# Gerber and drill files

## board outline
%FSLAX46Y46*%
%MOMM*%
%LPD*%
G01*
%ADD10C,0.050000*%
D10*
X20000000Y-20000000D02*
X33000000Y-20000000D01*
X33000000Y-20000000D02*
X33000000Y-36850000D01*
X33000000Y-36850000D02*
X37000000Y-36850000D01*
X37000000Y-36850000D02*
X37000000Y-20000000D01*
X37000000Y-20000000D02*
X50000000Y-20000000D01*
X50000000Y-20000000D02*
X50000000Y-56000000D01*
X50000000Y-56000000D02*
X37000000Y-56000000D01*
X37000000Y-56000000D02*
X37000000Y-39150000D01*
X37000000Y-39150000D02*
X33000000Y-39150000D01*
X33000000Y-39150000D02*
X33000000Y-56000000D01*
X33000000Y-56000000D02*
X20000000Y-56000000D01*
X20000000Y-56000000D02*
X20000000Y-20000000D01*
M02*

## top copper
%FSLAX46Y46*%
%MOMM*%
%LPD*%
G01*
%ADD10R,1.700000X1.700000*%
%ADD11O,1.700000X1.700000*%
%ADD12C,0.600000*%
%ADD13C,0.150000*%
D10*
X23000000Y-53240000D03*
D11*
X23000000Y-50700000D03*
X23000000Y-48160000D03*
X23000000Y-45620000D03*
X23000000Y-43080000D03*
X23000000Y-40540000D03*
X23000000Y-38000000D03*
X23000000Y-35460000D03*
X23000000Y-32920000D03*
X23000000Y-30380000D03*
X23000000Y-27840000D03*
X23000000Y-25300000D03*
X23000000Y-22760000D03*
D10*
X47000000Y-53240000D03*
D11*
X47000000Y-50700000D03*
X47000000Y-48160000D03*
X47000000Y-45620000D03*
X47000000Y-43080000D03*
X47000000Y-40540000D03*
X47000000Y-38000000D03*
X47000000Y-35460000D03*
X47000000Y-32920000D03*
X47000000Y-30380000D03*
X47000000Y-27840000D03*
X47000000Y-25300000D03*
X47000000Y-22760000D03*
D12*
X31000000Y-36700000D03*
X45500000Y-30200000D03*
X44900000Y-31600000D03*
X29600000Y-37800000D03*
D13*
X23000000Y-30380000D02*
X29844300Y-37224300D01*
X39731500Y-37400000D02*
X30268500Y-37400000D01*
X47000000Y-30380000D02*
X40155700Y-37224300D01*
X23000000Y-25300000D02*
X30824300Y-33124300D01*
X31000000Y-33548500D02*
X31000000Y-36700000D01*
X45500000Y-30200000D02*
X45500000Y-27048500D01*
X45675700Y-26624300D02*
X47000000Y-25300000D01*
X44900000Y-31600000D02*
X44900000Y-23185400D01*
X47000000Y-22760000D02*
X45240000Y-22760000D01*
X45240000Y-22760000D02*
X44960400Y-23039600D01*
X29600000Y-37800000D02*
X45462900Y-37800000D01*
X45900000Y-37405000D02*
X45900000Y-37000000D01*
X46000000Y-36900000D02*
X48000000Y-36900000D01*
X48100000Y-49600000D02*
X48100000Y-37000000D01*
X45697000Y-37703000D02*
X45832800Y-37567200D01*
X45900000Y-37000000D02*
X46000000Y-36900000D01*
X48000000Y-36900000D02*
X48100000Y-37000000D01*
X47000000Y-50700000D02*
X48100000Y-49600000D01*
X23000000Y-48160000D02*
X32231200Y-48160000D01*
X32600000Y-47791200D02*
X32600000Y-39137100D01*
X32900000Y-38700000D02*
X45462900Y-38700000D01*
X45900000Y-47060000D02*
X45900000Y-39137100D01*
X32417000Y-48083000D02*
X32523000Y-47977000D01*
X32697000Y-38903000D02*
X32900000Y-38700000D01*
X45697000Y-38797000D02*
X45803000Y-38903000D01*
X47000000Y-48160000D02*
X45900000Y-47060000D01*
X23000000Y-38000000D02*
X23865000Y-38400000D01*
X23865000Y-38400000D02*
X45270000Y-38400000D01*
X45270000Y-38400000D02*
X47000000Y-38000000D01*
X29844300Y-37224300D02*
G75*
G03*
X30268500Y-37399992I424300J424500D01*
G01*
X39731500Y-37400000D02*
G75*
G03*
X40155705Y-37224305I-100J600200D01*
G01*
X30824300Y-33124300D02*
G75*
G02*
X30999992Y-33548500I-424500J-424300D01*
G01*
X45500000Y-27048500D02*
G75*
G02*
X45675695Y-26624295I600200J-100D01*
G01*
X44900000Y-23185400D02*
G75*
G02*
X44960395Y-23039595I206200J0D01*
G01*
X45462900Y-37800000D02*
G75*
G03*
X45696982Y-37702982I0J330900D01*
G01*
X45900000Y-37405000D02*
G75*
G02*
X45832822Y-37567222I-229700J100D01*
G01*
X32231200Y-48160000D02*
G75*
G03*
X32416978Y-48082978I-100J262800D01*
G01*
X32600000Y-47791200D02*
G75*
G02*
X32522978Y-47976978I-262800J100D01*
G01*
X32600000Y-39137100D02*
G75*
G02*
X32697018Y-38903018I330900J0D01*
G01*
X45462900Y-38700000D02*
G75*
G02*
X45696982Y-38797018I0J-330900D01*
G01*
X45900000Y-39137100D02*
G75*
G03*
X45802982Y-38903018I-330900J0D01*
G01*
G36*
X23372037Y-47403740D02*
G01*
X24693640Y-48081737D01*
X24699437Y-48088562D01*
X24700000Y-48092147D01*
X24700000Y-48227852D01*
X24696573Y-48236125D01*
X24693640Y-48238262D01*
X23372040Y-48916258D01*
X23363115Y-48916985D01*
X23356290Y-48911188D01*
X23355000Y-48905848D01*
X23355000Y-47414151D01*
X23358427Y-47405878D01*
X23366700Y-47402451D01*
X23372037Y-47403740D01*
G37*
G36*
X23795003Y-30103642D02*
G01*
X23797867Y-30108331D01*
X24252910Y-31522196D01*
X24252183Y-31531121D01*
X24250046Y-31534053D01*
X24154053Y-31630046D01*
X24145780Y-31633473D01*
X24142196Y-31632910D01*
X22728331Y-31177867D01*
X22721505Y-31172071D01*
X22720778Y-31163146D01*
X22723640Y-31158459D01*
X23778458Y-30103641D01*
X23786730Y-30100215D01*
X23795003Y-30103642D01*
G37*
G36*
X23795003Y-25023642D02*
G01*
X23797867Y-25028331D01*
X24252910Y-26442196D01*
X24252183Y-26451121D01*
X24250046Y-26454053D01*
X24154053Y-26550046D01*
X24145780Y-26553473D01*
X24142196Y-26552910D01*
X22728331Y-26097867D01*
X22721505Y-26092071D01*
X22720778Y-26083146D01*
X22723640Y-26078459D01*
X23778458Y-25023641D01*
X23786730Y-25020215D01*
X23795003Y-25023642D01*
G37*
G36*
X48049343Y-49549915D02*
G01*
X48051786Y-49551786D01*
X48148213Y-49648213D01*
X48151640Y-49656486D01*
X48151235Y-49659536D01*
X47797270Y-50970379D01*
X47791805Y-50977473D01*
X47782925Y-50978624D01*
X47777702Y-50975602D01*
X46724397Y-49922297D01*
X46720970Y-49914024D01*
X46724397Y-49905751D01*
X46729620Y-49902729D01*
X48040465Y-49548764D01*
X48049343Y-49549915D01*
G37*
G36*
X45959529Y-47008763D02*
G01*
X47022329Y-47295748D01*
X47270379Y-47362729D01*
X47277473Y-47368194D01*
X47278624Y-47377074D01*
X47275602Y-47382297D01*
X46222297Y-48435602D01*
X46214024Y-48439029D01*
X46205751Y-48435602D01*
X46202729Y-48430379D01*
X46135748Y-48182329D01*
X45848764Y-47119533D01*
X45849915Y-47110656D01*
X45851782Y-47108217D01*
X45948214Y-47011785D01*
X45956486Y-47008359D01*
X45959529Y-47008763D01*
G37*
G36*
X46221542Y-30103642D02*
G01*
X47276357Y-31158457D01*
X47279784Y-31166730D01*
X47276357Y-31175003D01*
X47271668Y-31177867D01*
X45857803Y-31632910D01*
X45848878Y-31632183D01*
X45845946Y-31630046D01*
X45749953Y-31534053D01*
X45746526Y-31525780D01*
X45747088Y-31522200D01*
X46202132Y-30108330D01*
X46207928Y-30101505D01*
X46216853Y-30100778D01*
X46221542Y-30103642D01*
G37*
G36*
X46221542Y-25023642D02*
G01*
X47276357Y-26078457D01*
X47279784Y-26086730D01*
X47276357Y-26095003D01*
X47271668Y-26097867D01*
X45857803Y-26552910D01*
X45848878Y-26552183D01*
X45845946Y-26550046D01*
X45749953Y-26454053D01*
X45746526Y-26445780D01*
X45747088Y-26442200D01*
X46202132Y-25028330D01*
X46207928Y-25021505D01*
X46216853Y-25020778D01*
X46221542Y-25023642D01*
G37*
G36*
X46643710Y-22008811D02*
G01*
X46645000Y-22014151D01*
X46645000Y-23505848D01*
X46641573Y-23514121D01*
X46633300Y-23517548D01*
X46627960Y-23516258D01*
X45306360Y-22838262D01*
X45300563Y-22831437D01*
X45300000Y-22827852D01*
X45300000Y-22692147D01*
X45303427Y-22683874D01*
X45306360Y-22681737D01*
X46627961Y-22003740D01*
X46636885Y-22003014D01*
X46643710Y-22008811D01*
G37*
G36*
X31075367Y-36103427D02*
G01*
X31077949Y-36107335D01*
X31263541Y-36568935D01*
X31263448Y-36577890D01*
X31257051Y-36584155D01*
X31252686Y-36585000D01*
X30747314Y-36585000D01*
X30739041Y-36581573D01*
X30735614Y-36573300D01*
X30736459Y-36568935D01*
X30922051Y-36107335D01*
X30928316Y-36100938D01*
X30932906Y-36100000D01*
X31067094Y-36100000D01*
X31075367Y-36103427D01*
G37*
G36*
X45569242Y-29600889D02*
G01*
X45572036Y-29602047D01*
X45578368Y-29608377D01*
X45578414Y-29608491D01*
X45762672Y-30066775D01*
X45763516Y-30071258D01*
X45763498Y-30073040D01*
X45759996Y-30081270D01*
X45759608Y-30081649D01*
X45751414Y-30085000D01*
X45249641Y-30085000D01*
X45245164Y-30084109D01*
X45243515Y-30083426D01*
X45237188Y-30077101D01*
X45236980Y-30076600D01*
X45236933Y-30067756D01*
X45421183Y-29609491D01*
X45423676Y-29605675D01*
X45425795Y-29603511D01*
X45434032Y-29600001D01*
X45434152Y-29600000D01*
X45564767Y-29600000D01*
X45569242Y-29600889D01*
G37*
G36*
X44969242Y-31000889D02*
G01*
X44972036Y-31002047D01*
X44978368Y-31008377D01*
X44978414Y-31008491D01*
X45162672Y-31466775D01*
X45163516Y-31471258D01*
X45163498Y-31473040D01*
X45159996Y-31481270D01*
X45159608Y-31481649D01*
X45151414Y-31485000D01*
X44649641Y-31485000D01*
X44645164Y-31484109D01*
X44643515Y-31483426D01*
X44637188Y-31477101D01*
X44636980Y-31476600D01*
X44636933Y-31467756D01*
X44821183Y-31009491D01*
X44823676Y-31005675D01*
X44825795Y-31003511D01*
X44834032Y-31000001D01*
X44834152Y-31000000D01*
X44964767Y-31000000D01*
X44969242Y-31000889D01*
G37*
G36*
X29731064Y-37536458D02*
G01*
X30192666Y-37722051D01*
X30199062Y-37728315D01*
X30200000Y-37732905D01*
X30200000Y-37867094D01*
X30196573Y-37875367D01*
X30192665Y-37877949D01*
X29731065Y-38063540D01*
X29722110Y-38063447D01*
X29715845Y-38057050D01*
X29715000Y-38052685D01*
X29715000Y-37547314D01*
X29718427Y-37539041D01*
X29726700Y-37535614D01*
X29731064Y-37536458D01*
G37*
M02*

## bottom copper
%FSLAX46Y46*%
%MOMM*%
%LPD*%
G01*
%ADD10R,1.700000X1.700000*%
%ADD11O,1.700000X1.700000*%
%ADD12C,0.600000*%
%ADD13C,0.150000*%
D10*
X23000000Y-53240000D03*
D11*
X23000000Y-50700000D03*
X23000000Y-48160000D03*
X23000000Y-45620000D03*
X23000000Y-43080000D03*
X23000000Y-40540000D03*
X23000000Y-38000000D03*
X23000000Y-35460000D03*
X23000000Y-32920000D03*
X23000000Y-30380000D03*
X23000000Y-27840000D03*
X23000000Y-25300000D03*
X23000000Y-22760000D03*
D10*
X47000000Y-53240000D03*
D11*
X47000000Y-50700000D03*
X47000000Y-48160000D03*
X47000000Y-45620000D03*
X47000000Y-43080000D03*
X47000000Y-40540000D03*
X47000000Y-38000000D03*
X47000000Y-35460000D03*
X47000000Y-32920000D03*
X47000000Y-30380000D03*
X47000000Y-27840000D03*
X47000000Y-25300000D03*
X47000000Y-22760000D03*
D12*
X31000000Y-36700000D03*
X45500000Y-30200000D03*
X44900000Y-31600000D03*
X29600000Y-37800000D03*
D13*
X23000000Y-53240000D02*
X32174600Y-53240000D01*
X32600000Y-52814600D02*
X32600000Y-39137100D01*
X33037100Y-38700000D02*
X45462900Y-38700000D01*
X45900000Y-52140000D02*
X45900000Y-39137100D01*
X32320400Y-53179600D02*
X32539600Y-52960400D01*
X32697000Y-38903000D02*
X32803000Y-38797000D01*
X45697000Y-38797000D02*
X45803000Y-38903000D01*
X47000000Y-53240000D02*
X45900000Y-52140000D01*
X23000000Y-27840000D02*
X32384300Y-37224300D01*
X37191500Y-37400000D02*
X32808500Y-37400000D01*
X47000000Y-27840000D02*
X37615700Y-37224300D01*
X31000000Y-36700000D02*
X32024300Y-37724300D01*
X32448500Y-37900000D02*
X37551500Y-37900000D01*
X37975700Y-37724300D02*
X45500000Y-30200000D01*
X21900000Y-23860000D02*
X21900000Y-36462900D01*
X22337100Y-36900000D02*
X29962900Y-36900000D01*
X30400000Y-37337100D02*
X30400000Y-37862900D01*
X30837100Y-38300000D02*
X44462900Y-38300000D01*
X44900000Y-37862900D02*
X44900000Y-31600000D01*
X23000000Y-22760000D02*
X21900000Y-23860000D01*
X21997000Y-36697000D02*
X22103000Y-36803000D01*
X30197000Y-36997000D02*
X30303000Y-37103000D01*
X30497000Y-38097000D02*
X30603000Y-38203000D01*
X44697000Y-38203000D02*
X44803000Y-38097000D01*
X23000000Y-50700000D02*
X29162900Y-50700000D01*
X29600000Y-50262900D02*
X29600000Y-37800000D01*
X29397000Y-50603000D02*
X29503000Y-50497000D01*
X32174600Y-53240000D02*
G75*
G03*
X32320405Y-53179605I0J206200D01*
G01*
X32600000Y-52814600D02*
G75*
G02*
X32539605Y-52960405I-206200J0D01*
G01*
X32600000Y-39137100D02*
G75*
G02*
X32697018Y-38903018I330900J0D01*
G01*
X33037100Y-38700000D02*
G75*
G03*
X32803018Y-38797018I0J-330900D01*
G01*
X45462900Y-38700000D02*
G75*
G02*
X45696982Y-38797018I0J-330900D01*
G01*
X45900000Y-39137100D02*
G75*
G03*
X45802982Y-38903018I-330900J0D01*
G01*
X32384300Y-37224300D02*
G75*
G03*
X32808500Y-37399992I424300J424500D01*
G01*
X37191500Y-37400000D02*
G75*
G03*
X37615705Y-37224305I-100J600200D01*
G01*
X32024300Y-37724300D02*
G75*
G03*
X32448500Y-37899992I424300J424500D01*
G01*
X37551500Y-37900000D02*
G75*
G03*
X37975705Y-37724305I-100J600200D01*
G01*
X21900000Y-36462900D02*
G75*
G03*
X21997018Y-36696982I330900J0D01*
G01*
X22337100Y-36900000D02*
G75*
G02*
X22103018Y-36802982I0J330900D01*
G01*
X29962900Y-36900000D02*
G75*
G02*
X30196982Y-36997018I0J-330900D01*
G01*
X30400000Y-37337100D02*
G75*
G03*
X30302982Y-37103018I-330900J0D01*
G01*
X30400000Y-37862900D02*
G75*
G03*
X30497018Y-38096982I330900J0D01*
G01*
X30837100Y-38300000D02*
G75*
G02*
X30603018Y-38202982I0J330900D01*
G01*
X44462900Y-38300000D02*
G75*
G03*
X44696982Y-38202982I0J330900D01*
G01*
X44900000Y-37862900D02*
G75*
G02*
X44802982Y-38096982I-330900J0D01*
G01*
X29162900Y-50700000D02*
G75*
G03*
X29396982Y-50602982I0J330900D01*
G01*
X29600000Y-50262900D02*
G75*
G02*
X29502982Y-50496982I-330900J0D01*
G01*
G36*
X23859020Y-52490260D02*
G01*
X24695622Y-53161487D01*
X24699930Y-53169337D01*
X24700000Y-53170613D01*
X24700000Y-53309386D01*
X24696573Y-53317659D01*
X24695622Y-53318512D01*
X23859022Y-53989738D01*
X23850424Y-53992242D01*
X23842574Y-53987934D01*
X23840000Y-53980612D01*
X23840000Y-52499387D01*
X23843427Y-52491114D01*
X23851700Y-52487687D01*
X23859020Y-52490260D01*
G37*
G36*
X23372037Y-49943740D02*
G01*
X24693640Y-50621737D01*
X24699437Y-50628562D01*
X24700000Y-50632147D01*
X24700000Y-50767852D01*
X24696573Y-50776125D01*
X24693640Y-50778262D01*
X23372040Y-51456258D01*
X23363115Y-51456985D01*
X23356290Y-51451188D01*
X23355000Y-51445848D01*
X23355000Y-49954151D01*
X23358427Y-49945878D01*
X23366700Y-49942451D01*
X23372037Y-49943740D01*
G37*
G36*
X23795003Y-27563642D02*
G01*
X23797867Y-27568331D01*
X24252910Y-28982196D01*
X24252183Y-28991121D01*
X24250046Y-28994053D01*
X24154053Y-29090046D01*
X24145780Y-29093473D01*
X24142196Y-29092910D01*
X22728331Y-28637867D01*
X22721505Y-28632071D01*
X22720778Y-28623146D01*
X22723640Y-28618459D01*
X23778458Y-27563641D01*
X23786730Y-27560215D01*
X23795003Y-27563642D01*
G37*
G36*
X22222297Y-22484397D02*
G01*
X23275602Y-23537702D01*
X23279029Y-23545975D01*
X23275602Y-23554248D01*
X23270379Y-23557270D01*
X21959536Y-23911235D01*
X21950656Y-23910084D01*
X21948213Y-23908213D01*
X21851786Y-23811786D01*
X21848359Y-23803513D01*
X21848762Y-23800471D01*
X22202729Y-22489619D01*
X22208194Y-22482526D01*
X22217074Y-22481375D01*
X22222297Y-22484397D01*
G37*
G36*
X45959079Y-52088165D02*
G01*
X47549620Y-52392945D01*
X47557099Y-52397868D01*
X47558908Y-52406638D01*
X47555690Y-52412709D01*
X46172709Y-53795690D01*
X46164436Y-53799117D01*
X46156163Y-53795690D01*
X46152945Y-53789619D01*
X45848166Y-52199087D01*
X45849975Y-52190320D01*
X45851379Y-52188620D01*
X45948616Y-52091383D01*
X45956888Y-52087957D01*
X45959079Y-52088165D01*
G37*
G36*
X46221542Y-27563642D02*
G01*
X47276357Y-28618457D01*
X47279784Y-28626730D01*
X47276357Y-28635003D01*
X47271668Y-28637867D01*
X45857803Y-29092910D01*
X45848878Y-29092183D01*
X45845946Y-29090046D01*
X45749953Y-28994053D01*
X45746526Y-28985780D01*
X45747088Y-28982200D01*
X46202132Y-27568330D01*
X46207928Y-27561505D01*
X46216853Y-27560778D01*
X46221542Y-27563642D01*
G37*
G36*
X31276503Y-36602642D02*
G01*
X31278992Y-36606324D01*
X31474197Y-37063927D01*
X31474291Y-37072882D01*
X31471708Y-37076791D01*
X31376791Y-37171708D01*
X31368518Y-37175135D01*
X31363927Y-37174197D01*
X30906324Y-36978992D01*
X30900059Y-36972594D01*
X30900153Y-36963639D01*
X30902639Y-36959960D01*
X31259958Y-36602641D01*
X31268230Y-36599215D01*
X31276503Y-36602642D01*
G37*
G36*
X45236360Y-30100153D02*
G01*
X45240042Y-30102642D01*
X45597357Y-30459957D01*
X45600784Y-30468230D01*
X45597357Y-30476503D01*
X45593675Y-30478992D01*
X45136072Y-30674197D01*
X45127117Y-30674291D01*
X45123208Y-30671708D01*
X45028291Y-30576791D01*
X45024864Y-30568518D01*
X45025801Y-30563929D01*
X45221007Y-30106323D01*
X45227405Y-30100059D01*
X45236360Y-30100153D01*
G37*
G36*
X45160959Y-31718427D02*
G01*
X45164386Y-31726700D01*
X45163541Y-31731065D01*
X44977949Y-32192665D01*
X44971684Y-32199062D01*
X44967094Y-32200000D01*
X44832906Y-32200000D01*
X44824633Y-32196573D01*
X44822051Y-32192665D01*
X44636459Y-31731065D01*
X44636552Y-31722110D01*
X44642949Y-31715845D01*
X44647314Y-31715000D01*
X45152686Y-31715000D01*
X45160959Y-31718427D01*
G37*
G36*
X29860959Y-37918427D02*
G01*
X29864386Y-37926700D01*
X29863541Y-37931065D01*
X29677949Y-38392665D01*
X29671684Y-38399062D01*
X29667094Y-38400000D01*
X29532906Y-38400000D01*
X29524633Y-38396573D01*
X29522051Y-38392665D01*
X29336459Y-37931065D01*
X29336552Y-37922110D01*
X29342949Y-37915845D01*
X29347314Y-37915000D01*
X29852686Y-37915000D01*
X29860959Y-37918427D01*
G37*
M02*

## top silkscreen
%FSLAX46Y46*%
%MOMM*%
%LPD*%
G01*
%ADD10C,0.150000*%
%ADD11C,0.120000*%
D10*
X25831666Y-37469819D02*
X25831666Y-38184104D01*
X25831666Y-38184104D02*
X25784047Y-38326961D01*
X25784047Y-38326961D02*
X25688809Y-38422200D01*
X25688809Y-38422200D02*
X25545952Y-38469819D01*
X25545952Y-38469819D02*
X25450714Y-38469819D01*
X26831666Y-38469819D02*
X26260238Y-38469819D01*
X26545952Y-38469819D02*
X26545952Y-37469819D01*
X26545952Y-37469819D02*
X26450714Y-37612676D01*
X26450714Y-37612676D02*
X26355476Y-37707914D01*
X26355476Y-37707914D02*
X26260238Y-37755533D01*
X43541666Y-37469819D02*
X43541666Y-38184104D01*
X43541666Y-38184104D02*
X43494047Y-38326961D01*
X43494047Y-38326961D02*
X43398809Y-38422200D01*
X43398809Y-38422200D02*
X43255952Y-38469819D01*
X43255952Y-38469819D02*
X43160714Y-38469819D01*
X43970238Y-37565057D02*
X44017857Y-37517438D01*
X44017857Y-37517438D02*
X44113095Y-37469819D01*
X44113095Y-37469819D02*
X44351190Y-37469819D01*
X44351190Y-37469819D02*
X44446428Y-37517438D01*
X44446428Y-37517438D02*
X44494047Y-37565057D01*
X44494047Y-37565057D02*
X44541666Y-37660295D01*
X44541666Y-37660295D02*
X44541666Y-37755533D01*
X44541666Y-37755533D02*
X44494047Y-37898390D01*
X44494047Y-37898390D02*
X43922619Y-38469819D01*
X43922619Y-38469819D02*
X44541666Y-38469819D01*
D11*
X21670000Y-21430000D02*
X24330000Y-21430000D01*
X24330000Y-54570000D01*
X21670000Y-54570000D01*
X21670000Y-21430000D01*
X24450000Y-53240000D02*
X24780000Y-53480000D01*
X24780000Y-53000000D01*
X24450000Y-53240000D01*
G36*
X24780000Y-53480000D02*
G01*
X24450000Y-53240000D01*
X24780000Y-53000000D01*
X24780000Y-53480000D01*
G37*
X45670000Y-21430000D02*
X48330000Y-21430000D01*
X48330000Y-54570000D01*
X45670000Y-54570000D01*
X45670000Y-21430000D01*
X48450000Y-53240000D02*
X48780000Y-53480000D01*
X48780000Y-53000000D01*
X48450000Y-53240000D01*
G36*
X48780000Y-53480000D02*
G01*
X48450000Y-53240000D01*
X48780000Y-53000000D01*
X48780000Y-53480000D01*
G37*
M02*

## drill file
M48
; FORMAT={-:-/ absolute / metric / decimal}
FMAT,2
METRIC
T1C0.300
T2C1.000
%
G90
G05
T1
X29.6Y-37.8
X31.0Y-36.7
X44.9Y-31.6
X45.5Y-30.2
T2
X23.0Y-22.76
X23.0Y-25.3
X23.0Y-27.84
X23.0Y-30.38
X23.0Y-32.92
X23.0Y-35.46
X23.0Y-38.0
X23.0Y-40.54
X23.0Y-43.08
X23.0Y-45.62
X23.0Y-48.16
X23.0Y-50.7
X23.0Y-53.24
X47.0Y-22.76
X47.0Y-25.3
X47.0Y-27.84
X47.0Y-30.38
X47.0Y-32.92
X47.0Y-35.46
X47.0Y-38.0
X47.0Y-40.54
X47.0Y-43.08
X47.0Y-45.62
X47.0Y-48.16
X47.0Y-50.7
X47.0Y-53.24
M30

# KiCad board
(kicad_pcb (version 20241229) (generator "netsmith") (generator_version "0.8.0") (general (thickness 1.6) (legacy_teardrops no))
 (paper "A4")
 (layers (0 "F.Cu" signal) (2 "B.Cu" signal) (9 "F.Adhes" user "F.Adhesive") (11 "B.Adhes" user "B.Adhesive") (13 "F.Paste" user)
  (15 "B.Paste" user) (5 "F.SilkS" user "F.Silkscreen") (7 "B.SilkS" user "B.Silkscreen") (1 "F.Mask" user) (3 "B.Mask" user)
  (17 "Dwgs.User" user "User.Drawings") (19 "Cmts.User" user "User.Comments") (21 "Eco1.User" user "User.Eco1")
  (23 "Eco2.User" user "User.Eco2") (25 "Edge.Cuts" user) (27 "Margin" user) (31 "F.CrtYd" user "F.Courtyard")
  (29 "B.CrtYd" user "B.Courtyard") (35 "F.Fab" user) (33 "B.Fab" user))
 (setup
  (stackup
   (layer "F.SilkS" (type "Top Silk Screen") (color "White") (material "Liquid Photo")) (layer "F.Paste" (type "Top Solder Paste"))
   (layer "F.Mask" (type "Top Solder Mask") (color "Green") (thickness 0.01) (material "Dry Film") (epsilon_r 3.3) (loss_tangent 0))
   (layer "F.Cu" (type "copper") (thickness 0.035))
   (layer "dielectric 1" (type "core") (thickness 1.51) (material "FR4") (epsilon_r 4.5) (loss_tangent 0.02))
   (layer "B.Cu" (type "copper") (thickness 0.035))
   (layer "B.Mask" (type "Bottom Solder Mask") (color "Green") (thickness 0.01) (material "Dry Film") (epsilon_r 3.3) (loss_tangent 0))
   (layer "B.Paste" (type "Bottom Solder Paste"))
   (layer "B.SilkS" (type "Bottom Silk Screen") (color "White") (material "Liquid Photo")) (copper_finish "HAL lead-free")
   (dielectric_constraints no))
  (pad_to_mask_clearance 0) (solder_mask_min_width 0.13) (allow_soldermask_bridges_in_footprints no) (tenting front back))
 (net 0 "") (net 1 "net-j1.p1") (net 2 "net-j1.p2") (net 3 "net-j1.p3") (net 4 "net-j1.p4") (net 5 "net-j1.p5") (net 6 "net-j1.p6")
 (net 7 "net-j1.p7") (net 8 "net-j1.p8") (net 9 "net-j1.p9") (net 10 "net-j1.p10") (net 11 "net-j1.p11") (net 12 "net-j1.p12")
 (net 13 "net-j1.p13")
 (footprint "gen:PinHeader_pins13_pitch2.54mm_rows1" (layer "F.Cu") (at 23 53.24 180)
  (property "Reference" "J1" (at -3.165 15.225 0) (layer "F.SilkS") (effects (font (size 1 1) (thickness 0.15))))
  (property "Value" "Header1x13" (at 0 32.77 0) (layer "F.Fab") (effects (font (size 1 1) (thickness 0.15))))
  (pad "1" thru_hole rect (at 0 0 180) (size 1.7 1.7) (drill 1) (layers "*.Cu" "*.Mask") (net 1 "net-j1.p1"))
  (pad "2" thru_hole oval (at 0 2.54 180) (size 1.7 1.7) (drill 1) (layers "*.Cu" "*.Mask") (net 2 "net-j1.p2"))
  (pad "3" thru_hole oval (at 0 5.08 180) (size 1.7 1.7) (drill 1) (layers "*.Cu" "*.Mask") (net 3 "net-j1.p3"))
  (pad "4" thru_hole oval (at 0 7.62 180) (size 1.7 1.7) (drill 1) (layers "*.Cu" "*.Mask") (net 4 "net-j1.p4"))
  (pad "5" thru_hole oval (at 0 10.16 180) (size 1.7 1.7) (drill 1) (layers "*.Cu" "*.Mask") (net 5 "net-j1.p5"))
  (pad "6" thru_hole oval (at 0 12.7 180) (size 1.7 1.7) (drill 1) (layers "*.Cu" "*.Mask") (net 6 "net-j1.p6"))
  (pad "7" thru_hole oval (at 0 15.24 180) (size 1.7 1.7) (drill 1) (layers "*.Cu" "*.Mask") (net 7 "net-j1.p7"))
  (pad "8" thru_hole oval (at 0 17.78 180) (size 1.7 1.7) (drill 1) (layers "*.Cu" "*.Mask") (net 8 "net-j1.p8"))
  (pad "9" thru_hole oval (at 0 20.32 180) (size 1.7 1.7) (drill 1) (layers "*.Cu" "*.Mask") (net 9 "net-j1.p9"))
  (pad "10" thru_hole oval (at 0 22.86 180) (size 1.7 1.7) (drill 1) (layers "*.Cu" "*.Mask") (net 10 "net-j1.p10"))
  (pad "11" thru_hole oval (at 0 25.4 180) (size 1.7 1.7) (drill 1) (layers "*.Cu" "*.Mask") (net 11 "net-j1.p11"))
  (pad "12" thru_hole oval (at 0 27.94 180) (size 1.7 1.7) (drill 1) (layers "*.Cu" "*.Mask") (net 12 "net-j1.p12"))
  (pad "13" thru_hole oval (at 0 30.48 180) (size 1.7 1.7) (drill 1) (layers "*.Cu" "*.Mask") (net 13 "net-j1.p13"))
  (fp_rect (start -1.33 -1.33) (end 1.33 31.81) (stroke (width 0.12) (type solid)) (fill no) (layer "F.SilkS"))
  (fp_poly (pts (xy -1.45 0) (xy -1.78 -0.24) (xy -1.78 0.24)) (stroke (width 0.12) (type solid)) (fill solid) (layer "F.SilkS")))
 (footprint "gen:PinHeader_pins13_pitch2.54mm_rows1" (layer "F.Cu") (at 47 53.24 180)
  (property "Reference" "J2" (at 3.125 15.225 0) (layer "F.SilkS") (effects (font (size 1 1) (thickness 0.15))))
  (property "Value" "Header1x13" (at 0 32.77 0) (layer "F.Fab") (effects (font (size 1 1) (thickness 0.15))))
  (pad "1" thru_hole rect (at 0 0 180) (size 1.7 1.7) (drill 1) (layers "*.Cu" "*.Mask") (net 1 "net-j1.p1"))
  (pad "2" thru_hole oval (at 0 2.54 180) (size 1.7 1.7) (drill 1) (layers "*.Cu" "*.Mask") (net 2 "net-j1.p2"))
  (pad "3" thru_hole oval (at 0 5.08 180) (size 1.7 1.7) (drill 1) (layers "*.Cu" "*.Mask") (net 3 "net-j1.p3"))
  (pad "4" thru_hole oval (at 0 7.62 180) (size 1.7 1.7) (drill 1) (layers "*.Cu" "*.Mask") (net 4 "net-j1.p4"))
  (pad "5" thru_hole oval (at 0 10.16 180) (size 1.7 1.7) (drill 1) (layers "*.Cu" "*.Mask") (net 5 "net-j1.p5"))
  (pad "6" thru_hole oval (at 0 12.7 180) (size 1.7 1.7) (drill 1) (layers "*.Cu" "*.Mask") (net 6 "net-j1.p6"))
  (pad "7" thru_hole oval (at 0 15.24 180) (size 1.7 1.7) (drill 1) (layers "*.Cu" "*.Mask") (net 7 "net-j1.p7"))
  (pad "8" thru_hole oval (at 0 17.78 180) (size 1.7 1.7) (drill 1) (layers "*.Cu" "*.Mask") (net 8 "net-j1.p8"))
  (pad "9" thru_hole oval (at 0 20.32 180) (size 1.7 1.7) (drill 1) (layers "*.Cu" "*.Mask") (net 9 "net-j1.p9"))
  (pad "10" thru_hole oval (at 0 22.86 180) (size 1.7 1.7) (drill 1) (layers "*.Cu" "*.Mask") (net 10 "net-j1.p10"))
  (pad "11" thru_hole oval (at 0 25.4 180) (size 1.7 1.7) (drill 1) (layers "*.Cu" "*.Mask") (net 11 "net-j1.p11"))
  (pad "12" thru_hole oval (at 0 27.94 180) (size 1.7 1.7) (drill 1) (layers "*.Cu" "*.Mask") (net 12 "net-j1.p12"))
  (pad "13" thru_hole oval (at 0 30.48 180) (size 1.7 1.7) (drill 1) (layers "*.Cu" "*.Mask") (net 13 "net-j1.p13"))
  (fp_rect (start -1.33 -1.33) (end 1.33 31.81) (stroke (width 0.12) (type solid)) (fill no) (layer "F.SilkS"))
  (fp_poly (pts (xy -1.45 0) (xy -1.78 -0.24) (xy -1.78 0.24)) (stroke (width 0.12) (type solid)) (fill solid) (layer "F.SilkS")))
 (segment (start 23 53.24) (end 32.1746 53.24) (width 0.15) (layer "B.Cu") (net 1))
 (segment (start 32.6 52.8146) (end 32.6 39.1371) (width 0.15) (layer "B.Cu") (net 1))
 (segment (start 33.0371 38.7) (end 45.4629 38.7) (width 0.15) (layer "B.Cu") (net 1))
 (segment (start 45.9 52.14) (end 45.9 39.1371) (width 0.15) (layer "B.Cu") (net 1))
 (segment (start 32.3204 53.1796) (end 32.5396 52.9604) (width 0.15) (layer "B.Cu") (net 1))
 (segment (start 32.697 38.903) (end 32.803 38.797) (width 0.15) (layer "B.Cu") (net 1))
 (segment (start 45.697 38.797) (end 45.803 38.903) (width 0.15) (layer "B.Cu") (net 1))
 (segment (start 47 53.24) (end 45.9 52.14) (width 0.15) (layer "B.Cu") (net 1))
 (segment (start 23 30.38) (end 29.8443 37.2243) (width 0.15) (layer "F.Cu") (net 10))
 (segment (start 39.7315 37.4) (end 30.2685 37.4) (width 0.15) (layer "F.Cu") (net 10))
 (segment (start 47 30.38) (end 40.1557 37.2243) (width 0.15) (layer "F.Cu") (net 10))
 (segment (start 23 27.84) (end 32.3843 37.2243) (width 0.15) (layer "B.Cu") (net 11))
 (segment (start 37.1915 37.4) (end 32.8085 37.4) (width 0.15) (layer "B.Cu") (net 11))
 (segment (start 47 27.84) (end 37.6157 37.2243) (width 0.15) (layer "B.Cu") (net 11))
 (segment (start 23 25.3) (end 30.8243 33.1243) (width 0.15) (layer "F.Cu") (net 12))
 (segment (start 31 33.5485) (end 31 36.7) (width 0.15) (layer "F.Cu") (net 12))
 (segment (start 31 36.7) (end 32.0243 37.7243) (width 0.15) (layer "B.Cu") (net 12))
 (segment (start 32.4485 37.9) (end 37.5515 37.9) (width 0.15) (layer "B.Cu") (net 12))
 (segment (start 37.9757 37.7243) (end 45.5 30.2) (width 0.15) (layer "B.Cu") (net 12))
 (segment (start 45.5 30.2) (end 45.5 27.0485) (width 0.15) (layer "F.Cu") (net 12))
 (segment (start 45.6757 26.6243) (end 47 25.3) (width 0.15) (layer "F.Cu") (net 12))
 (segment (start 21.9 23.86) (end 21.9 36.4629) (width 0.15) (layer "B.Cu") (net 13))
 (segment (start 22.3371 36.9) (end 29.9629 36.9) (width 0.15) (layer "B.Cu") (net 13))
 (segment (start 30.4 37.3371) (end 30.4 37.8629) (width 0.15) (layer "B.Cu") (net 13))
 (segment (start 30.8371 38.3) (end 44.4629 38.3) (width 0.15) (layer "B.Cu") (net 13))
 (segment (start 44.9 37.8629) (end 44.9 31.6) (width 0.15) (layer "B.Cu") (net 13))
 (segment (start 44.9 31.6) (end 44.9 23.1854) (width 0.15) (layer "F.Cu") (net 13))
 (segment (start 47 22.76) (end 45.24 22.76) (width 0.15) (layer "F.Cu") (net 13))
 (segment (start 23 22.76) (end 21.9 23.86) (width 0.15) (layer "B.Cu") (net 13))
 (segment (start 21.997 36.697) (end 22.103 36.803) (width 0.15) (layer "B.Cu") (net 13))
 (segment (start 30.197 36.997) (end 30.303 37.103) (width 0.15) (layer "B.Cu") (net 13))
 (segment (start 30.497 38.097) (end 30.603 38.203) (width 0.15) (layer "B.Cu") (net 13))
 (segment (start 44.697 38.203) (end 44.803 38.097) (width 0.15) (layer "B.Cu") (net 13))
 (segment (start 45.24 22.76) (end 44.9604 23.0396) (width 0.15) (layer "F.Cu") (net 13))
 (segment (start 23 50.7) (end 29.1629 50.7) (width 0.15) (layer "B.Cu") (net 2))
 (segment (start 29.6 50.2629) (end 29.6 37.8) (width 0.15) (layer "B.Cu") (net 2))
 (segment (start 29.6 37.8) (end 45.4629 37.8) (width 0.15) (layer "F.Cu") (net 2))
 (segment (start 45.9 37.405) (end 45.9 37) (width 0.15) (layer "F.Cu") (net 2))
 (segment (start 46 36.9) (end 48 36.9) (width 0.15) (layer "F.Cu") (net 2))
 (segment (start 48.1 49.6) (end 48.1 37) (width 0.15) (layer "F.Cu") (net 2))
 (segment (start 29.397 50.603) (end 29.503 50.497) (width 0.15) (layer "B.Cu") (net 2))
 (segment (start 45.697 37.703) (end 45.8328 37.5672) (width 0.15) (layer "F.Cu") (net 2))
 (segment (start 45.9 37) (end 46 36.9) (width 0.15) (layer "F.Cu") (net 2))
 (segment (start 48 36.9) (end 48.1 37) (width 0.15) (layer "F.Cu") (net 2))
 (segment (start 47 50.7) (end 48.1 49.6) (width 0.15) (layer "F.Cu") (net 2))
 (segment (start 23 48.16) (end 32.2312 48.16) (width 0.15) (layer "F.Cu") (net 3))
 (segment (start 32.6 47.7912) (end 32.6 39.1371) (width 0.15) (layer "F.Cu") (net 3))
 (segment (start 32.9 38.7) (end 45.4629 38.7) (width 0.15) (layer "F.Cu") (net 3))
 (segment (start 45.9 47.06) (end 45.9 39.1371) (width 0.15) (layer "F.Cu") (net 3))
 (segment (start 32.417 48.083) (end 32.523 47.977) (width 0.15) (layer "F.Cu") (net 3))
 (segment (start 32.697 38.903) (end 32.9 38.7) (width 0.15) (layer "F.Cu") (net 3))
 (segment (start 45.697 38.797) (end 45.803 38.903) (width 0.15) (layer "F.Cu") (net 3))
 (segment (start 47 48.16) (end 45.9 47.06) (width 0.15) (layer "F.Cu") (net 3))
 (segment (start 23 38) (end 23.865 38.4) (width 0.15) (layer "F.Cu") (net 7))
 (segment (start 23.865 38.4) (end 45.27 38.4) (width 0.15) (layer "F.Cu") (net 7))
 (segment (start 45.27 38.4) (end 47 38) (width 0.15) (layer "F.Cu") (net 7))
 (arc (start 32.1746 53.24) (mid 32.2535 53.2243) (end 32.3204 53.1796) (width 0.15) (layer "B.Cu") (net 1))
 (arc (start 32.6 52.8146) (mid 32.5843 52.8935) (end 32.5396 52.9604) (width 0.15) (layer "B.Cu") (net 1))
 (arc (start 32.6 39.1371) (mid 32.6252 39.0104) (end 32.697 38.903) (width 0.15) (layer "B.Cu") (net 1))
 (arc (start 33.0371 38.7) (mid 32.9104 38.7252) (end 32.803 38.797) (width 0.15) (layer "B.Cu") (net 1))
 (arc (start 45.4629 38.7) (mid 45.5896 38.7252) (end 45.697 38.797) (width 0.15) (layer "B.Cu") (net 1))
 (arc (start 45.9 39.1371) (mid 45.8748 39.0104) (end 45.803 38.903) (width 0.15) (layer "B.Cu") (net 1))
 (arc (start 29.8443 37.2243) (mid 30.0389 37.3543) (end 30.2685 37.4) (width 0.15) (layer "F.Cu") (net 10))
 (arc (start 39.7315 37.4) (mid 39.9611 37.3543) (end 40.1557 37.2243) (width 0.15) (layer "F.Cu") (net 10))
 (arc (start 32.3843 37.2243) (mid 32.5789 37.3543) (end 32.8085 37.4) (width 0.15) (layer "B.Cu") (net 11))
 (arc (start 37.1915 37.4) (mid 37.4211 37.3543) (end 37.6157 37.2243) (width 0.15) (layer "B.Cu") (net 11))
 (arc (start 30.8243 33.1243) (mid 30.9543 33.3189) (end 31 33.5485) (width 0.15) (layer "F.Cu") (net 12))
 (arc (start 32.0243 37.7243) (mid 32.2189 37.8543) (end 32.4485 37.9) (width 0.15) (layer "B.Cu") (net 12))
 (arc (start 37.5515 37.9) (mid 37.7811 37.8543) (end 37.9757 37.7243) (width 0.15) (layer "B.Cu") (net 12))
 (arc (start 45.5 27.0485) (mid 45.5457 26.8189) (end 45.6757 26.6243) (width 0.15) (layer "F.Cu") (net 12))
 (arc (start 21.9 36.4629) (mid 21.9252 36.5896) (end 21.997 36.697) (width 0.15) (layer "B.Cu") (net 13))
 (arc (start 22.3371 36.9) (mid 22.2104 36.8748) (end 22.103 36.803) (width 0.15) (layer "B.Cu") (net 13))
 (arc (start 29.9629 36.9) (mid 30.0896 36.9252) (end 30.197 36.997) (width 0.15) (layer "B.Cu") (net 13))
 (arc (start 30.4 37.3371) (mid 30.3748 37.2104) (end 30.303 37.103) (width 0.15) (layer "B.Cu") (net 13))
 (arc (start 30.4 37.8629) (mid 30.4252 37.9896) (end 30.497 38.097) (width 0.15) (layer "B.Cu") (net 13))
 (arc (start 30.8371 38.3) (mid 30.7104 38.2748) (end 30.603 38.203) (width 0.15) (layer "B.Cu") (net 13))
 (arc (start 44.4629 38.3) (mid 44.5896 38.2748) (end 44.697 38.203) (width 0.15) (layer "B.Cu") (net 13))
 (arc (start 44.9 37.8629) (mid 44.8748 37.9896) (end 44.803 38.097) (width 0.15) (layer "B.Cu") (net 13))
 (arc (start 44.9 23.1854) (mid 44.9157 23.1065) (end 44.9604 23.0396) (width 0.15) (layer "F.Cu") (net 13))
 (arc (start 29.1629 50.7) (mid 29.2896 50.6748) (end 29.397 50.603) (width 0.15) (layer "B.Cu") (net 2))
 (arc (start 29.6 50.2629) (mid 29.5748 50.3896) (end 29.503 50.497) (width 0.15) (layer "B.Cu") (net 2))
 (arc (start 45.4629 37.8) (mid 45.5896 37.7748) (end 45.697 37.703) (width 0.15) (layer "F.Cu") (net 2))
 (arc (start 45.9 37.405) (mid 45.8825 37.4928) (end 45.8328 37.5672) (width 0.15) (layer "F.Cu") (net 2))
 (arc (start 32.2312 48.16) (mid 32.3317 48.14) (end 32.417 48.083) (width 0.15) (layer "F.Cu") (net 3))
 (arc (start 32.6 47.7912) (mid 32.58 47.8917) (end 32.523 47.977) (width 0.15) (layer "F.Cu") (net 3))
 (arc (start 32.6 39.1371) (mid 32.6252 39.0104) (end 32.697 38.903) (width 0.15) (layer "F.Cu") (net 3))
 (arc (start 45.4629 38.7) (mid 45.5896 38.7252) (end 45.697 38.797) (width 0.15) (layer "F.Cu") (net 3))
 (arc (start 45.9 39.1371) (mid 45.8748 39.0104) (end 45.803 38.903) (width 0.15) (layer "F.Cu") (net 3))
 (via (at 31 36.7) (size 0.6) (drill 0.3) (layers "F.Cu" "B.Cu") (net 12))
 (via (at 45.5 30.2) (size 0.6) (drill 0.3) (layers "F.Cu" "B.Cu") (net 12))
 (via (at 44.9 31.6) (size 0.6) (drill 0.3) (layers "F.Cu" "B.Cu") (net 13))
 (via (at 29.6 37.8) (size 0.6) (drill 0.3) (layers "F.Cu" "B.Cu") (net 2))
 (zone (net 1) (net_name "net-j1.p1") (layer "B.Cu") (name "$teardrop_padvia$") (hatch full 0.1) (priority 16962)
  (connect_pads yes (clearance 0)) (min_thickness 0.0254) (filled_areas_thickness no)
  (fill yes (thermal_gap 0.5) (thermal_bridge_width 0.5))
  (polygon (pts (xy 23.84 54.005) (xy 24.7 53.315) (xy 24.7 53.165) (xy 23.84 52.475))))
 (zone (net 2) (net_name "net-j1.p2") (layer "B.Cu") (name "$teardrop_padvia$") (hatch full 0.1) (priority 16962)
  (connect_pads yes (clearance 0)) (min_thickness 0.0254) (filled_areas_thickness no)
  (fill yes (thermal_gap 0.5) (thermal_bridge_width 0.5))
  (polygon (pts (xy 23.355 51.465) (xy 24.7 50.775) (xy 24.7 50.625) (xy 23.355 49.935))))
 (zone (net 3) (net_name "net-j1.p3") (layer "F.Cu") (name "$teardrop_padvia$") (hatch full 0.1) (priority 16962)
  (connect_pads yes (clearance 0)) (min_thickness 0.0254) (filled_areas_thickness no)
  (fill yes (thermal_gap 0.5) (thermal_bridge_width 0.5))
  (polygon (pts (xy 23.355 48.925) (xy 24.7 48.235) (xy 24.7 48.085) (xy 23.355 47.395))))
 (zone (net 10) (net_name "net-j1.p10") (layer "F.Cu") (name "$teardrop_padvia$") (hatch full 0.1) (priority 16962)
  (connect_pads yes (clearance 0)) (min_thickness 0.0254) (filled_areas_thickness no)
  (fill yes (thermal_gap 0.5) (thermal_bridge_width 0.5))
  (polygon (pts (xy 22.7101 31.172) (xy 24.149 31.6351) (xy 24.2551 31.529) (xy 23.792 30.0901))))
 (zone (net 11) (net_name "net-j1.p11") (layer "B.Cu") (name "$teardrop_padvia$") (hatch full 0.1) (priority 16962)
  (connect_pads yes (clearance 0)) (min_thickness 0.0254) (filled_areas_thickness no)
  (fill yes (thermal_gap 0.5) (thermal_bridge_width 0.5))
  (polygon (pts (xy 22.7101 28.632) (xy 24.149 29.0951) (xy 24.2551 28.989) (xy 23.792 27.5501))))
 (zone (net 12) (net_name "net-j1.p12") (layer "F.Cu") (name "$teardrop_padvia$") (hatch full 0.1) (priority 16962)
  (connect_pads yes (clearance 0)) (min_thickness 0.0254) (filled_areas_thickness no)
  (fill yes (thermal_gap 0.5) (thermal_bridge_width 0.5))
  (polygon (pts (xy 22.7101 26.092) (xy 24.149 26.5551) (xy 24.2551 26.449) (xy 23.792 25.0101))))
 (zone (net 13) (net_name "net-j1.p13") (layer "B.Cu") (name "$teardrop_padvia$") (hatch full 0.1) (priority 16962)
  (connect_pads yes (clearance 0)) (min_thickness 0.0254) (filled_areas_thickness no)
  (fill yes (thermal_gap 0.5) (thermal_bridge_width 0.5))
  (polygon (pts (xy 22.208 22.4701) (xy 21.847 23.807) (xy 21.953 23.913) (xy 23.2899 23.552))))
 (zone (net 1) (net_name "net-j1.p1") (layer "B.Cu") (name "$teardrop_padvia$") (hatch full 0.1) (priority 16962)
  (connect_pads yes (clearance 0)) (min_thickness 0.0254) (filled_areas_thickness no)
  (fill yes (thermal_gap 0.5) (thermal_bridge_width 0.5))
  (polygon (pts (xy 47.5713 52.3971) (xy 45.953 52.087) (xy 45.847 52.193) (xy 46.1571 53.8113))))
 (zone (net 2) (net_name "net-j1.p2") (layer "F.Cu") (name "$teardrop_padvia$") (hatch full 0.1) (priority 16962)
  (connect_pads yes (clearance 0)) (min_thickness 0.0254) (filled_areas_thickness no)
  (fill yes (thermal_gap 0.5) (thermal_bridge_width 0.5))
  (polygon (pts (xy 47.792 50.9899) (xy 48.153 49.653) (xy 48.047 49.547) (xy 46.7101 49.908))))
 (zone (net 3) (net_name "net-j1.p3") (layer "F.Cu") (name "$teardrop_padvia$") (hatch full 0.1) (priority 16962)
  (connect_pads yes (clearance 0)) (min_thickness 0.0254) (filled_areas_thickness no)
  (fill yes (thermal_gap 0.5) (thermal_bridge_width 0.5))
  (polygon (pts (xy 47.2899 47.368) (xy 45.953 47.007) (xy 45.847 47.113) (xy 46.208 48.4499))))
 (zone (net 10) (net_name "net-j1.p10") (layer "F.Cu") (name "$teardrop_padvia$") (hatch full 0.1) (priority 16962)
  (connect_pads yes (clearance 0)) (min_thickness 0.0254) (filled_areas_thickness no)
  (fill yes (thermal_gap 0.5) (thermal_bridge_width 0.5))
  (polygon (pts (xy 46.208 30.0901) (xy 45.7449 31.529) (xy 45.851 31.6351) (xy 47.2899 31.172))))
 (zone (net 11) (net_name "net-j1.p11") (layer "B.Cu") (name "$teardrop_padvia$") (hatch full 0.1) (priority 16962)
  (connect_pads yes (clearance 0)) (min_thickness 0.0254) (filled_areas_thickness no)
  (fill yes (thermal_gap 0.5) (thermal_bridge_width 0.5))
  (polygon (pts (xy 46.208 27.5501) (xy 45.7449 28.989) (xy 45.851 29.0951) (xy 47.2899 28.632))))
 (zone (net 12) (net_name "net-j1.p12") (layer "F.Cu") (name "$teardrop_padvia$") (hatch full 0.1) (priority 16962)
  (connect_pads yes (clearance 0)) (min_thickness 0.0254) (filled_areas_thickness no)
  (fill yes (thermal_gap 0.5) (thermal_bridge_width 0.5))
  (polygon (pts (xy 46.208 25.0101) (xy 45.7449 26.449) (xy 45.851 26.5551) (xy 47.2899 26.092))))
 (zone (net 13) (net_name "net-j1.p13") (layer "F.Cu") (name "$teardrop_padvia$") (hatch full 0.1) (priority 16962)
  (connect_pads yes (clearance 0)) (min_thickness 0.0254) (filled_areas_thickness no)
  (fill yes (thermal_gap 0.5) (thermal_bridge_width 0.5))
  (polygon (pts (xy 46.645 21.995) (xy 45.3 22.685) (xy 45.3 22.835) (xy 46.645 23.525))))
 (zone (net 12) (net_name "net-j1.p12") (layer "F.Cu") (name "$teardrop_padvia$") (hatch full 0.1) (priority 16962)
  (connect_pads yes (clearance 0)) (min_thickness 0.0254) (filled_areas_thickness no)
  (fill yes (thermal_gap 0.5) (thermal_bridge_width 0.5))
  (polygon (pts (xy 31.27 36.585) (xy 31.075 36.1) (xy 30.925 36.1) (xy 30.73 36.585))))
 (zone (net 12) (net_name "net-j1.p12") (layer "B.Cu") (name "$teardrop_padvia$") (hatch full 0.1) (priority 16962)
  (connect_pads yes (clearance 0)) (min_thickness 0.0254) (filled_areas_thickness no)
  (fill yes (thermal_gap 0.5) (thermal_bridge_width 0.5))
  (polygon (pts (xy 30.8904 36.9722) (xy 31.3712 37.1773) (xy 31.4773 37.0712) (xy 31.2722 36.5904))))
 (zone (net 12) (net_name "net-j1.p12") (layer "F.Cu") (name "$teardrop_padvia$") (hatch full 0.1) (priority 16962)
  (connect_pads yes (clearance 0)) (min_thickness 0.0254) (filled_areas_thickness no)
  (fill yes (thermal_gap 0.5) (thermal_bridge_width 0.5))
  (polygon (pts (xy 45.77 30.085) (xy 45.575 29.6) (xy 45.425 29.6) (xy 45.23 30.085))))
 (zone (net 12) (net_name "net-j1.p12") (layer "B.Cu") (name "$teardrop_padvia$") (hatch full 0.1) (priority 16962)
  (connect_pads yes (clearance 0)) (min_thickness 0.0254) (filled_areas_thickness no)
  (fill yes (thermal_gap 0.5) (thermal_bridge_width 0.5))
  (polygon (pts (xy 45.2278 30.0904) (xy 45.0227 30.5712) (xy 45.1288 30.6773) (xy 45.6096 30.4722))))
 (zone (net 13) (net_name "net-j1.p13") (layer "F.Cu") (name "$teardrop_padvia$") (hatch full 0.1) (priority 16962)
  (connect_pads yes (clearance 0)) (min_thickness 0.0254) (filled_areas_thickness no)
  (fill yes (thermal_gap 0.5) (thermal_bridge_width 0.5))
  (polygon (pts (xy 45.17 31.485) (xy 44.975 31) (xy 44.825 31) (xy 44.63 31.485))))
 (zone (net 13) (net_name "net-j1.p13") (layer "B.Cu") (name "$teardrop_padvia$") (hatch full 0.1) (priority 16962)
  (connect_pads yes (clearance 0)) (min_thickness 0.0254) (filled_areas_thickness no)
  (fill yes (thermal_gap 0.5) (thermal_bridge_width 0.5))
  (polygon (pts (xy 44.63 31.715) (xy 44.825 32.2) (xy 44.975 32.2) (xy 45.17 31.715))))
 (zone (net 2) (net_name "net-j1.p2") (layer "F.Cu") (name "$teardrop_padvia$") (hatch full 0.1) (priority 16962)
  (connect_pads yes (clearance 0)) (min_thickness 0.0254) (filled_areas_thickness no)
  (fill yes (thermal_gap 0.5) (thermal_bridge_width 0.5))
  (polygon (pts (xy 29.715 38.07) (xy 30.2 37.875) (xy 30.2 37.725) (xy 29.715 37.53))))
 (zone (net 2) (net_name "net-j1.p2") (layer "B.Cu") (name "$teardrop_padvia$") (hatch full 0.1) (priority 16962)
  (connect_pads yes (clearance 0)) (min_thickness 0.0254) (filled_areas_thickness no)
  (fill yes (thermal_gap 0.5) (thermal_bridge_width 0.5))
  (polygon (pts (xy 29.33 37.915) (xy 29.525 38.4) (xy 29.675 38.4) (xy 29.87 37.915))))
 (gr_line (start 20 20) (end 33 20) (stroke (width 0.05) (type default)) (layer "Edge.Cuts"))
 (gr_line (start 33 20) (end 33 36.85) (stroke (width 0.05) (type default)) (layer "Edge.Cuts"))
 (gr_line (start 33 36.85) (end 37 36.85) (stroke (width 0.05) (type default)) (layer "Edge.Cuts"))
 (gr_line (start 37 36.85) (end 37 20) (stroke (width 0.05) (type default)) (layer "Edge.Cuts"))
 (gr_line (start 37 20) (end 50 20) (stroke (width 0.05) (type default)) (layer "Edge.Cuts"))
 (gr_line (start 50 20) (end 50 56) (stroke (width 0.05) (type default)) (layer "Edge.Cuts"))
 (gr_line (start 50 56) (end 37 56) (stroke (width 0.05) (type default)) (layer "Edge.Cuts"))
 (gr_line (start 37 56) (end 37 39.15) (stroke (width 0.05) (type default)) (layer "Edge.Cuts"))
 (gr_line (start 37 39.15) (end 33 39.15) (stroke (width 0.05) (type default)) (layer "Edge.Cuts"))
 (gr_line (start 33 39.15) (end 33 56) (stroke (width 0.05) (type default)) (layer "Edge.Cuts"))
 (gr_line (start 33 56) (end 20 56) (stroke (width 0.05) (type default)) (layer "Edge.Cuts"))
 (gr_line (start 20 56) (end 20 20) (stroke (width 0.05) (type default)) (layer "Edge.Cuts")))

